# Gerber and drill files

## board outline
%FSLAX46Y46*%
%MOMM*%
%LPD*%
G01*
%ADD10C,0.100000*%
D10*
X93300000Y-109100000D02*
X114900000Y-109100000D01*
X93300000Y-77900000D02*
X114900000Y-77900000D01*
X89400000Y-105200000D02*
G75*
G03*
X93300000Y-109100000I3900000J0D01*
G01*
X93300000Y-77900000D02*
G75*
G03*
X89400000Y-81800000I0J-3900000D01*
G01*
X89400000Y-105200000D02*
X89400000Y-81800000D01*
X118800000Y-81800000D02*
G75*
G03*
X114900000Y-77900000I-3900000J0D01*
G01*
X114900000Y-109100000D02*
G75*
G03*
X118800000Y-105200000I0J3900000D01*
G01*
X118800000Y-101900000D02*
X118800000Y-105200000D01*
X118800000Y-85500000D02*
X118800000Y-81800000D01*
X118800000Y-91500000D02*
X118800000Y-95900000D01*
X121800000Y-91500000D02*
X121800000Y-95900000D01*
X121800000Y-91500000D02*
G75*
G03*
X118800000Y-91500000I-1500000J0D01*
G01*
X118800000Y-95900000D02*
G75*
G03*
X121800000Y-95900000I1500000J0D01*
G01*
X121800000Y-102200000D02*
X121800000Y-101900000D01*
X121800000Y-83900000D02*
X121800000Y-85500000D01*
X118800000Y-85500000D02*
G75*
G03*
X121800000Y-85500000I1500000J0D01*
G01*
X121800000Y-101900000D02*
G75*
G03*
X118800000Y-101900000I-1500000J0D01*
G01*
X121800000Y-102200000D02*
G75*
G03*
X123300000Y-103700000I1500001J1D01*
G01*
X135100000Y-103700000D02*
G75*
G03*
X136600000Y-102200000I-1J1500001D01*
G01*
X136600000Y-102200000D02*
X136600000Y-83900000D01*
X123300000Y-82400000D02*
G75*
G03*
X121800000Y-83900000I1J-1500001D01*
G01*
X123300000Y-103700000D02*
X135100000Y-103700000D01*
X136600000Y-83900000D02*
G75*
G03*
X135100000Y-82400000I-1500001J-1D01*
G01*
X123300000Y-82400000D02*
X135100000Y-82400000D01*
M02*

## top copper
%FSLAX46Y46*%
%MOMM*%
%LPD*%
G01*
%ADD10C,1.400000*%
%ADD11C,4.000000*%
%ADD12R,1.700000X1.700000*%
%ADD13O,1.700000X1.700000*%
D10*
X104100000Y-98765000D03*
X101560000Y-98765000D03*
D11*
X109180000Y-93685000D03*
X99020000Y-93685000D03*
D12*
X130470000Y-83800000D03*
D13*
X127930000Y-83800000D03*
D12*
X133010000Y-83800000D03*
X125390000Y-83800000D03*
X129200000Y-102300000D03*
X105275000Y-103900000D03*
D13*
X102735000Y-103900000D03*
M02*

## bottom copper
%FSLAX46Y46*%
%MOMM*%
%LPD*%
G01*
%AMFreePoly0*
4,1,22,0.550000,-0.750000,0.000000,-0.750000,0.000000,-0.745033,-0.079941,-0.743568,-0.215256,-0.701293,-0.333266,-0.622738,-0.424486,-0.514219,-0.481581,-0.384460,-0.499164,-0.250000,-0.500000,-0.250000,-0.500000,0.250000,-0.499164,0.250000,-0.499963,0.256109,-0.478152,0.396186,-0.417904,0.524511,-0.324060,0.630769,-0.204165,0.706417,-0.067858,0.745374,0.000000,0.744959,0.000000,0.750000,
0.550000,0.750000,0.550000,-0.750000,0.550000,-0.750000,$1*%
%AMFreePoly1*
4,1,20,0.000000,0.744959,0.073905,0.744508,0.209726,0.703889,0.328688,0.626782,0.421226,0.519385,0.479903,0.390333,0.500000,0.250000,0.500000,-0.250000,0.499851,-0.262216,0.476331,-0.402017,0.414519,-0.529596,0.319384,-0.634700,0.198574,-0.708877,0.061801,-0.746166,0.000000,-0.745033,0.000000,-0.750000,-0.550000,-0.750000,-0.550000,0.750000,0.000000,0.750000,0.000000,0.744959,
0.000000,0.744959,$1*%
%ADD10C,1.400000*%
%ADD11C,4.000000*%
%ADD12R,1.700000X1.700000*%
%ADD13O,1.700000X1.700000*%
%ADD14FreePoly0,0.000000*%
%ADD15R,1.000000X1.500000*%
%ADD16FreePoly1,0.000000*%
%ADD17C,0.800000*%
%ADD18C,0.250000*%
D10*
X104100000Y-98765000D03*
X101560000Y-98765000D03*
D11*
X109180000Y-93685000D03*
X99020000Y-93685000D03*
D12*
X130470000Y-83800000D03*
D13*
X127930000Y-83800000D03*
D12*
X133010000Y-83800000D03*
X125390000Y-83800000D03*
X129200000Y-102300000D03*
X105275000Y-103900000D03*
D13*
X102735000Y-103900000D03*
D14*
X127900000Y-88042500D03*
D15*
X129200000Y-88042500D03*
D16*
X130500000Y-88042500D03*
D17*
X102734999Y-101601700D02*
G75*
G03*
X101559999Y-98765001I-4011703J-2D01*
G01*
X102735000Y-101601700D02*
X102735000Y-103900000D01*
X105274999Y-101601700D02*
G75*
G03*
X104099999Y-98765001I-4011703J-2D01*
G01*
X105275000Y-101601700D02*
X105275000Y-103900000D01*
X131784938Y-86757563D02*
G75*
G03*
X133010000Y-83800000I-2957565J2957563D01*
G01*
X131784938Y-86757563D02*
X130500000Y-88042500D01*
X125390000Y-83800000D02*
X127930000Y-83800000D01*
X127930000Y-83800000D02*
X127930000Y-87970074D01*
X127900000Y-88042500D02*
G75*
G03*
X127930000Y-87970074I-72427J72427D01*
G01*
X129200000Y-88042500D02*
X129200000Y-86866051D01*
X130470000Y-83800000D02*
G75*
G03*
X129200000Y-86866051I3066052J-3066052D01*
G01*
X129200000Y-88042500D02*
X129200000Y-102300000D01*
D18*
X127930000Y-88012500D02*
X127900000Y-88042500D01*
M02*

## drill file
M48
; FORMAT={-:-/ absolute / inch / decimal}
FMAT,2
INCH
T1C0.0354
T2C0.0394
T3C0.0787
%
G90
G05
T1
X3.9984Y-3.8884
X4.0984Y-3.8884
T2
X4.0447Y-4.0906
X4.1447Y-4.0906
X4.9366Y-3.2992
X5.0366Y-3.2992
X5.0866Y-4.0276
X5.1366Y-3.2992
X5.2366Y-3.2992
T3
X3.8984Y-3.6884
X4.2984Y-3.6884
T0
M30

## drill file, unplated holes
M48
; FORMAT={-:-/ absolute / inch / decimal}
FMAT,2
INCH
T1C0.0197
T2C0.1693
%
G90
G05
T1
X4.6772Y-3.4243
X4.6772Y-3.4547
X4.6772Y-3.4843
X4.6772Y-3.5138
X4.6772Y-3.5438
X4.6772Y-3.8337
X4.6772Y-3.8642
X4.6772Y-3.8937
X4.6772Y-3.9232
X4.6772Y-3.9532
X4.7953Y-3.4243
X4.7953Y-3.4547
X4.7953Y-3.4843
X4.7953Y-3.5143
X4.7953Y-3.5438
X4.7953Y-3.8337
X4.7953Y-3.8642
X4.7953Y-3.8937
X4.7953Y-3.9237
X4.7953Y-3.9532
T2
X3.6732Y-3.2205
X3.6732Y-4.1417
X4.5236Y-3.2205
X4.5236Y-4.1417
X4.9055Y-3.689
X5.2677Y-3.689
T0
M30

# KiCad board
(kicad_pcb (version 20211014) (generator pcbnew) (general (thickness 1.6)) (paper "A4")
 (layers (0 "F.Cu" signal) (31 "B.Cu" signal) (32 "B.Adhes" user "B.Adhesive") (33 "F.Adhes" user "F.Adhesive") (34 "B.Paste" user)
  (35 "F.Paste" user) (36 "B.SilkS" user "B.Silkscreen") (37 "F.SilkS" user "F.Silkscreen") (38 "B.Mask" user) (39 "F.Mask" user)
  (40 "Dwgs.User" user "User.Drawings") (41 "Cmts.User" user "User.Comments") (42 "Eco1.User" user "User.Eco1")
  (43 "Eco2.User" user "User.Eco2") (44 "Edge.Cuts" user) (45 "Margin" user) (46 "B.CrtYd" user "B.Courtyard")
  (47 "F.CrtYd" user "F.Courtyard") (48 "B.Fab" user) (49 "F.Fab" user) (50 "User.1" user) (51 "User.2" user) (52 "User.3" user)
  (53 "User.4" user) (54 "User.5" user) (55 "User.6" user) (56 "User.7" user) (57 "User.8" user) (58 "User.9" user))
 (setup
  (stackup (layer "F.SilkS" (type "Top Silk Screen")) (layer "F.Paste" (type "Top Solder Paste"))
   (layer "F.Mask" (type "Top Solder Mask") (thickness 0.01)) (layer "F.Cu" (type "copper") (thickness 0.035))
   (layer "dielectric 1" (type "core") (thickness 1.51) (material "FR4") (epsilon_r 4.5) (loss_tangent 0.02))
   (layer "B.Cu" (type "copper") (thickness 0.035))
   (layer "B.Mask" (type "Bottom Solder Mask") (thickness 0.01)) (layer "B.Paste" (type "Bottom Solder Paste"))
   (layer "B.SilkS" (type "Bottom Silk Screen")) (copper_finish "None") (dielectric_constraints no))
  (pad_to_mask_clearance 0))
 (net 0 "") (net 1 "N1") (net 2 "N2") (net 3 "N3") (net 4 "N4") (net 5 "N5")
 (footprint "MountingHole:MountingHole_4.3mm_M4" (layer "F.Cu") (at 93.3 105.2)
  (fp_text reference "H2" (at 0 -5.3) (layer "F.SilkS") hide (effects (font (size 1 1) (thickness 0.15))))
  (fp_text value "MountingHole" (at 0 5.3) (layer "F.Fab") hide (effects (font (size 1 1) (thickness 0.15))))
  (pad "" np_thru_hole circle (at 0 0) (size 4.3 4.3) (drill 4.3) (layers *.Cu *.Mask)))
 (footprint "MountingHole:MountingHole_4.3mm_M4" (layer "F.Cu") (at 133.8 93.7)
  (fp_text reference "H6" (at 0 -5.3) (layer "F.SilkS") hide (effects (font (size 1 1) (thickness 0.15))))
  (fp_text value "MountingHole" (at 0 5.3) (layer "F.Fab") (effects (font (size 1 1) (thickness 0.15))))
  (pad "" np_thru_hole circle (at 0 0) (size 4.3 4.3) (drill 4.3) (layers *.Cu *.Mask)))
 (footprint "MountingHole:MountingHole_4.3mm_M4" (layer "F.Cu") (at 93.3 81.8)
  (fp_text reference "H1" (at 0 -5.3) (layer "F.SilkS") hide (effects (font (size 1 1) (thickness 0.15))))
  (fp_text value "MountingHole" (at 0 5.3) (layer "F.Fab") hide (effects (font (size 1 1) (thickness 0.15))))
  (pad "" np_thru_hole circle (at 0 0) (size 4.3 4.3) (drill 4.3) (layers *.Cu *.Mask)))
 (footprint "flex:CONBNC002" (layer "F.Cu") (at 104.1 93.685)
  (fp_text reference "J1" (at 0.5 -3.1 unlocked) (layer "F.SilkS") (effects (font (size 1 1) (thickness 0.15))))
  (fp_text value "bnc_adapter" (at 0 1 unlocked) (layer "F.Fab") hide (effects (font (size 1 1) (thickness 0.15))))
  (pad "1" thru_hole circle (at 0 5.08 90) (size 1.4 1.4) (drill 0.9) (layers *.Cu *.Mask) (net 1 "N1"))
  (pad "2" thru_hole circle (at -2.54 5.08 90) (size 1.4 1.4) (drill 0.9) (layers *.Cu *.Mask) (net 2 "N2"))
  (pad "~" thru_hole circle (at -5.08 0 90) (size 4 4) (drill 2) (layers *.Cu *.Mask))
  (pad "~" thru_hole circle (at 5.08 0 90) (size 4 4) (drill 2) (layers *.Cu *.Mask)))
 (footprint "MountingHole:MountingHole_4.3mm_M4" (layer "F.Cu") (at 114.9 105.2)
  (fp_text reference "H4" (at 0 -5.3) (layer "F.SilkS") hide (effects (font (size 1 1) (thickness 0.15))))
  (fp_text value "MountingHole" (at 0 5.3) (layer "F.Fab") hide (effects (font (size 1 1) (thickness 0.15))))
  (pad "" np_thru_hole circle (at 0 0) (size 4.3 4.3) (drill 4.3) (layers *.Cu *.Mask)))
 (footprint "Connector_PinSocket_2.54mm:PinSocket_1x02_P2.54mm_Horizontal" (layer "F.Cu") (at 130.47 83.8 -90)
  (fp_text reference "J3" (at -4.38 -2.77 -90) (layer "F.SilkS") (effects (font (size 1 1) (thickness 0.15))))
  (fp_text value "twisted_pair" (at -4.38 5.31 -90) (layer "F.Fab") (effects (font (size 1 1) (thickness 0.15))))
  (pad "1" thru_hole rect (at 0 0 270) (size 1.7 1.7) (drill 1) (layers *.Cu *.Mask) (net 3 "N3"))
  (pad "2" thru_hole oval (at 0 2.54 270) (size 1.7 1.7) (drill 1) (layers *.Cu *.Mask) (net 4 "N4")))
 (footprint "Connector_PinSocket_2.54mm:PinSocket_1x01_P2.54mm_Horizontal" (layer "F.Cu") (at 133.01 83.8 -90)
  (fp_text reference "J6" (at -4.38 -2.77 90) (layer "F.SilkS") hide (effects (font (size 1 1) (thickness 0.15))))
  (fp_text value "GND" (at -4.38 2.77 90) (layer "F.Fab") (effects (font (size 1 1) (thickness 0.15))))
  (pad "1" thru_hole rect (at 0 0 270) (size 1.7 1.7) (drill 1) (layers *.Cu *.Mask) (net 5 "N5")))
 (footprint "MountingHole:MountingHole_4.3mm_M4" (layer "F.Cu") (at 124.6 93.7)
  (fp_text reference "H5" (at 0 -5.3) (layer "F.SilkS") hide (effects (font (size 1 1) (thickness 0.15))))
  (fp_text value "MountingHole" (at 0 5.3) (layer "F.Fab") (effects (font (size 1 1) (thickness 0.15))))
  (pad "" np_thru_hole circle (at 0 0) (size 4.3 4.3) (drill 4.3) (layers *.Cu *.Mask)))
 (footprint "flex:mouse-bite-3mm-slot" (layer "F.Cu") (at 120.3 98.9 90)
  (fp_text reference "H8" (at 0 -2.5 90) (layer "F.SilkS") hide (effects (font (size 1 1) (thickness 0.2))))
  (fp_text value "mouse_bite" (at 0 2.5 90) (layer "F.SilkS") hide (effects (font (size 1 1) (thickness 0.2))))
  (pad "" np_thru_hole circle locked (at 0 -1.5 90) (size 0.5 0.5) (drill 0.5) (layers *.Cu *.Mask))
  (pad "" np_thru_hole circle locked (at 0.75 1.5 90) (size 0.5 0.5) (drill 0.5) (layers *.Cu *.Mask))
  (pad "" np_thru_hole circle locked (at 1.524 -1.5 90) (size 0.5 0.5) (drill 0.5) (layers *.Cu *.Mask))
  (pad "" np_thru_hole circle locked (at -0.75 -1.5 90) (size 0.5 0.5) (drill 0.5) (layers *.Cu *.Mask))
  (pad "" np_thru_hole circle locked (at 0 1.5 90) (size 0.5 0.5) (drill 0.5) (layers *.Cu *.Mask))
  (pad "" np_thru_hole circle locked (at -1.512 1.5 90) (size 0.5 0.5) (drill 0.5) (layers *.Cu *.Mask))
  (pad "" np_thru_hole circle locked (at -1.512 -1.5 90) (size 0.5 0.5) (drill 0.5) (layers *.Cu *.Mask))
  (pad "" np_thru_hole circle locked (at 1.524 1.5 90) (size 0.5 0.5) (drill 0.5) (layers *.Cu *.Mask))
  (pad "" np_thru_hole circle locked (at -0.762 1.5 90) (size 0.5 0.5) (drill 0.5) (layers *.Cu *.Mask))
  (pad "" np_thru_hole circle locked (at 0.75 -1.5 90) (size 0.5 0.5) (drill 0.5) (layers *.Cu *.Mask)))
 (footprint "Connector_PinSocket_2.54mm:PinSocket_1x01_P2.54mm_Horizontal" (layer "F.Cu") (at 125.39 83.8 -90)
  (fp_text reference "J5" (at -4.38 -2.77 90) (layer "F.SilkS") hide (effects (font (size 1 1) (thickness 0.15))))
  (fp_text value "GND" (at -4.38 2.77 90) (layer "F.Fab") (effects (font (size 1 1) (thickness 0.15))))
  (pad "1" thru_hole rect (at 0 0 270) (size 1.7 1.7) (drill 1) (layers *.Cu *.Mask) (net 4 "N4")))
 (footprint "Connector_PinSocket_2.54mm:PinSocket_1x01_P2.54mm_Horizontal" (layer "F.Cu") (at 129.2 102.3 90)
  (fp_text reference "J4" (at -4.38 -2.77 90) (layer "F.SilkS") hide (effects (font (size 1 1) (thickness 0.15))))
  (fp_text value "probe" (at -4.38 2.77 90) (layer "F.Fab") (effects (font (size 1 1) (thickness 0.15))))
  (pad "1" thru_hole rect (at 0 0 90) (size 1.7 1.7) (drill 1) (layers *.Cu *.Mask) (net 3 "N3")))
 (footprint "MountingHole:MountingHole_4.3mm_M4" (layer "F.Cu") (at 114.9 81.8)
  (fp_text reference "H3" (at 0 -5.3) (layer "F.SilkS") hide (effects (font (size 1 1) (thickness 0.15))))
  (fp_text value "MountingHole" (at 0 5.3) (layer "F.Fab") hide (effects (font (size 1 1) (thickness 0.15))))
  (pad "" np_thru_hole circle (at 0 0) (size 4.3 4.3) (drill 4.3) (layers *.Cu *.Mask)))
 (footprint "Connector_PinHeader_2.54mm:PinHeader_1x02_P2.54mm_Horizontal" (layer "F.Cu") (at 105.275 103.9 -90)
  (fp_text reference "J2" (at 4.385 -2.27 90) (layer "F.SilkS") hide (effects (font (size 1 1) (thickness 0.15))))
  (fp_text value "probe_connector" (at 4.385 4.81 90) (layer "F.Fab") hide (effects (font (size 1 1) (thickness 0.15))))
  (pad "1" thru_hole rect (at 0 0 270) (size 1.7 1.7) (drill 1) (layers *.Cu *.Mask) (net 1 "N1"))
  (pad "2" thru_hole oval (at 0 2.54 270) (size 1.7 1.7) (drill 1) (layers *.Cu *.Mask) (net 2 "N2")))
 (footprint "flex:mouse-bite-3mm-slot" (layer "F.Cu") (at 120.3 88.5 90)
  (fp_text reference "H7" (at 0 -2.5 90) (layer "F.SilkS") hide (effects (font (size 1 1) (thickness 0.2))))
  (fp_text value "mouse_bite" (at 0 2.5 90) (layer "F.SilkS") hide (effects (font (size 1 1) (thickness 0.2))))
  (pad "" np_thru_hole circle locked (at -0.762 1.5 90) (size 0.5 0.5) (drill 0.5) (layers *.Cu *.Mask))
  (pad "" np_thru_hole circle locked (at 0.75 1.5 90) (size 0.5 0.5) (drill 0.5) (layers *.Cu *.Mask))
  (pad "" np_thru_hole circle locked (at -1.512 -1.5 90) (size 0.5 0.5) (drill 0.5) (layers *.Cu *.Mask))
  (pad "" np_thru_hole circle locked (at 0 -1.5 90) (size 0.5 0.5) (drill 0.5) (layers *.Cu *.Mask))
  (pad "" np_thru_hole circle locked (at 0 1.5 90) (size 0.5 0.5) (drill 0.5) (layers *.Cu *.Mask))
  (pad "" np_thru_hole circle locked (at -1.512 1.5 90) (size 0.5 0.5) (drill 0.5) (layers *.Cu *.Mask))
  (pad "" np_thru_hole circle locked (at -0.75 -1.5 90) (size 0.5 0.5) (drill 0.5) (layers *.Cu *.Mask))
  (pad "" np_thru_hole circle locked (at 1.524 -1.5 90) (size 0.5 0.5) (drill 0.5) (layers *.Cu *.Mask))
  (pad "" np_thru_hole circle locked (at 1.524 1.5 90) (size 0.5 0.5) (drill 0.5) (layers *.Cu *.Mask))
  (pad "" np_thru_hole circle locked (at 0.75 -1.5 90) (size 0.5 0.5) (drill 0.5) (layers *.Cu *.Mask)))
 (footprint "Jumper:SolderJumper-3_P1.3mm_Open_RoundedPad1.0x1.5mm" (layer "B.Cu") (at 129.2 88.0425)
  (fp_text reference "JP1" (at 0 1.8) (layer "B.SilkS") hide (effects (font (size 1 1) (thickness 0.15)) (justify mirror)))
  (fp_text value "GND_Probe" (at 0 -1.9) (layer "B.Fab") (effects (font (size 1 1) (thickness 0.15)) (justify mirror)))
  (pad "1" smd custom (at -1.3 0) (size 1 0.5) (layers "B.Cu" "B.Mask") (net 4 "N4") (zone_connect 2)
   (options (clearance outline) (anchor rect)) (primitives))
  (pad "2" smd rect (at 0 0) (size 1 1.5) (layers "B.Cu" "B.Mask") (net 3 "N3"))
  (pad "3" smd custom (at 1.3 0) (size 1 0.5) (layers "B.Cu" "B.Mask") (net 5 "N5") (zone_connect 2)
   (options (clearance outline) (anchor rect)) (primitives)))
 (gr_arc (start 123.3 103.7) (mid 122.23934 103.26066) (end 121.8 102.2) (layer "Edge.Cuts") (width 0.1))
 (gr_arc (start 118.8 101.9) (mid 120.3 100.4) (end 121.8 101.9) (layer "Edge.Cuts") (width 0.1))
 (gr_arc (start 121.8 85.5) (mid 120.3 87) (end 118.8 85.5) (layer "Edge.Cuts") (width 0.1))
 (gr_arc (start 136.6 102.2) (mid 136.16066 103.26066) (end 135.1 103.7) (layer "Edge.Cuts") (width 0.1))
 (gr_line (start 93.3 109.1) (end 114.9 109.1) (layer "Edge.Cuts") (width 0.1))
 (gr_line (start 121.8 83.9) (end 121.8 85.5) (layer "Edge.Cuts") (width 0.1))
 (gr_arc (start 118.8 105.2) (mid 117.657716 107.957716) (end 114.9 109.1) (layer "Edge.Cuts") (width 0.1))
 (gr_line (start 136.6 102.2) (end 136.6 83.9) (layer "Edge.Cuts") (width 0.1))
 (gr_arc (start 121.8 83.9) (mid 122.23934 82.83934) (end 123.3 82.4) (layer "Edge.Cuts") (width 0.1))
 (gr_arc (start 114.9 77.9) (mid 117.657716 79.042284) (end 118.8 81.8) (layer "Edge.Cuts") (width 0.1))
 (gr_line (start 123.3 103.7) (end 135.1 103.7) (layer "Edge.Cuts") (width 0.1))
 (gr_arc (start 89.4 81.8) (mid 90.542284 79.042284) (end 93.3 77.9) (layer "Edge.Cuts") (width 0.1))
 (gr_line (start 89.4 105.2) (end 89.4 81.8) (layer "Edge.Cuts") (width 0.1))
 (gr_arc (start 135.1 82.4) (mid 136.16066 82.83934) (end 136.6 83.9) (layer "Edge.Cuts") (width 0.1))
 (gr_line (start 121.8 102.2) (end 121.8 101.9) (layer "Edge.Cuts") (width 0.1))
 (gr_arc (start 121.8 95.9) (mid 120.3 97.4) (end 118.8 95.9) (layer "Edge.Cuts") (width 0.1))
 (gr_line (start 121.8 91.5) (end 121.8 95.9) (layer "Edge.Cuts") (width 0.1))
 (gr_line (start 118.8 85.5) (end 118.8 81.8) (layer "Edge.Cuts") (width 0.1))
 (gr_line (start 118.8 91.5) (end 118.8 95.9) (layer "Edge.Cuts") (width 0.1))
 (gr_arc (start 93.3 109.1) (mid 90.542284 107.957716) (end 89.4 105.2) (layer "Edge.Cuts") (width 0.1))
 (gr_line (start 123.3 82.4) (end 135.1 82.4) (layer "Edge.Cuts") (width 0.1))
 (gr_line (start 93.3 77.9) (end 114.9 77.9) (layer "Edge.Cuts") (width 0.1))
 (gr_line (start 118.8 101.9) (end 118.8 105.2) (layer "Edge.Cuts") (width 0.1))
 (gr_arc (start 118.8 91.5) (mid 120.3 90) (end 121.8 91.5) (layer "Edge.Cuts") (width 0.1))
 (segment (start 105.275 101.6017) (end 105.275 103.9) (width 0.8) (layer "B.Cu") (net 1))
 (arc (start 104.1 98.765) (mid 104.969627 100.066489) (end 105.275 101.6017) (width 0.8) (layer "B.Cu") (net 1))
 (segment (start 102.735 101.6017) (end 102.735 103.9) (width 0.8) (layer "B.Cu") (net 2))
 (arc (start 101.56 98.765) (mid 102.429627 100.066489) (end 102.735 101.6017) (width 0.8) (layer "B.Cu") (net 2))
 (segment (start 129.2 88.0425) (end 129.2 102.3) (width 0.8) (layer "B.Cu") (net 3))
 (segment (start 129.2 88.0425) (end 129.2 86.866051) (width 0.8) (layer "B.Cu") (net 3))
 (arc (start 129.2 86.866051) (mid 129.530062 85.206717) (end 130.47 83.8) (width 0.8) (layer "B.Cu") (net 3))
 (segment (start 127.93 83.8) (end 127.93 87.970074) (width 0.8) (layer "B.Cu") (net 4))
 (segment (start 127.93 88.0125) (end 127.9 88.0425) (width 0.25) (layer "B.Cu") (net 4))
 (segment (start 125.39 83.8) (end 127.93 83.8) (width 0.8) (layer "B.Cu") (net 4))
 (arc (start 127.93 87.970074) (mid 127.922203 88.009271) (end 127.9 88.0425) (width 0.8) (layer "B.Cu") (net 4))
 (segment (start 131.784938 86.757563) (end 130.5 88.0425) (width 0.8) (layer "B.Cu") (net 5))
 (arc (start 133.01 83.8) (mid 132.691617 85.400621) (end 131.784938 86.757563) (width 0.8) (layer "B.Cu") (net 5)))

